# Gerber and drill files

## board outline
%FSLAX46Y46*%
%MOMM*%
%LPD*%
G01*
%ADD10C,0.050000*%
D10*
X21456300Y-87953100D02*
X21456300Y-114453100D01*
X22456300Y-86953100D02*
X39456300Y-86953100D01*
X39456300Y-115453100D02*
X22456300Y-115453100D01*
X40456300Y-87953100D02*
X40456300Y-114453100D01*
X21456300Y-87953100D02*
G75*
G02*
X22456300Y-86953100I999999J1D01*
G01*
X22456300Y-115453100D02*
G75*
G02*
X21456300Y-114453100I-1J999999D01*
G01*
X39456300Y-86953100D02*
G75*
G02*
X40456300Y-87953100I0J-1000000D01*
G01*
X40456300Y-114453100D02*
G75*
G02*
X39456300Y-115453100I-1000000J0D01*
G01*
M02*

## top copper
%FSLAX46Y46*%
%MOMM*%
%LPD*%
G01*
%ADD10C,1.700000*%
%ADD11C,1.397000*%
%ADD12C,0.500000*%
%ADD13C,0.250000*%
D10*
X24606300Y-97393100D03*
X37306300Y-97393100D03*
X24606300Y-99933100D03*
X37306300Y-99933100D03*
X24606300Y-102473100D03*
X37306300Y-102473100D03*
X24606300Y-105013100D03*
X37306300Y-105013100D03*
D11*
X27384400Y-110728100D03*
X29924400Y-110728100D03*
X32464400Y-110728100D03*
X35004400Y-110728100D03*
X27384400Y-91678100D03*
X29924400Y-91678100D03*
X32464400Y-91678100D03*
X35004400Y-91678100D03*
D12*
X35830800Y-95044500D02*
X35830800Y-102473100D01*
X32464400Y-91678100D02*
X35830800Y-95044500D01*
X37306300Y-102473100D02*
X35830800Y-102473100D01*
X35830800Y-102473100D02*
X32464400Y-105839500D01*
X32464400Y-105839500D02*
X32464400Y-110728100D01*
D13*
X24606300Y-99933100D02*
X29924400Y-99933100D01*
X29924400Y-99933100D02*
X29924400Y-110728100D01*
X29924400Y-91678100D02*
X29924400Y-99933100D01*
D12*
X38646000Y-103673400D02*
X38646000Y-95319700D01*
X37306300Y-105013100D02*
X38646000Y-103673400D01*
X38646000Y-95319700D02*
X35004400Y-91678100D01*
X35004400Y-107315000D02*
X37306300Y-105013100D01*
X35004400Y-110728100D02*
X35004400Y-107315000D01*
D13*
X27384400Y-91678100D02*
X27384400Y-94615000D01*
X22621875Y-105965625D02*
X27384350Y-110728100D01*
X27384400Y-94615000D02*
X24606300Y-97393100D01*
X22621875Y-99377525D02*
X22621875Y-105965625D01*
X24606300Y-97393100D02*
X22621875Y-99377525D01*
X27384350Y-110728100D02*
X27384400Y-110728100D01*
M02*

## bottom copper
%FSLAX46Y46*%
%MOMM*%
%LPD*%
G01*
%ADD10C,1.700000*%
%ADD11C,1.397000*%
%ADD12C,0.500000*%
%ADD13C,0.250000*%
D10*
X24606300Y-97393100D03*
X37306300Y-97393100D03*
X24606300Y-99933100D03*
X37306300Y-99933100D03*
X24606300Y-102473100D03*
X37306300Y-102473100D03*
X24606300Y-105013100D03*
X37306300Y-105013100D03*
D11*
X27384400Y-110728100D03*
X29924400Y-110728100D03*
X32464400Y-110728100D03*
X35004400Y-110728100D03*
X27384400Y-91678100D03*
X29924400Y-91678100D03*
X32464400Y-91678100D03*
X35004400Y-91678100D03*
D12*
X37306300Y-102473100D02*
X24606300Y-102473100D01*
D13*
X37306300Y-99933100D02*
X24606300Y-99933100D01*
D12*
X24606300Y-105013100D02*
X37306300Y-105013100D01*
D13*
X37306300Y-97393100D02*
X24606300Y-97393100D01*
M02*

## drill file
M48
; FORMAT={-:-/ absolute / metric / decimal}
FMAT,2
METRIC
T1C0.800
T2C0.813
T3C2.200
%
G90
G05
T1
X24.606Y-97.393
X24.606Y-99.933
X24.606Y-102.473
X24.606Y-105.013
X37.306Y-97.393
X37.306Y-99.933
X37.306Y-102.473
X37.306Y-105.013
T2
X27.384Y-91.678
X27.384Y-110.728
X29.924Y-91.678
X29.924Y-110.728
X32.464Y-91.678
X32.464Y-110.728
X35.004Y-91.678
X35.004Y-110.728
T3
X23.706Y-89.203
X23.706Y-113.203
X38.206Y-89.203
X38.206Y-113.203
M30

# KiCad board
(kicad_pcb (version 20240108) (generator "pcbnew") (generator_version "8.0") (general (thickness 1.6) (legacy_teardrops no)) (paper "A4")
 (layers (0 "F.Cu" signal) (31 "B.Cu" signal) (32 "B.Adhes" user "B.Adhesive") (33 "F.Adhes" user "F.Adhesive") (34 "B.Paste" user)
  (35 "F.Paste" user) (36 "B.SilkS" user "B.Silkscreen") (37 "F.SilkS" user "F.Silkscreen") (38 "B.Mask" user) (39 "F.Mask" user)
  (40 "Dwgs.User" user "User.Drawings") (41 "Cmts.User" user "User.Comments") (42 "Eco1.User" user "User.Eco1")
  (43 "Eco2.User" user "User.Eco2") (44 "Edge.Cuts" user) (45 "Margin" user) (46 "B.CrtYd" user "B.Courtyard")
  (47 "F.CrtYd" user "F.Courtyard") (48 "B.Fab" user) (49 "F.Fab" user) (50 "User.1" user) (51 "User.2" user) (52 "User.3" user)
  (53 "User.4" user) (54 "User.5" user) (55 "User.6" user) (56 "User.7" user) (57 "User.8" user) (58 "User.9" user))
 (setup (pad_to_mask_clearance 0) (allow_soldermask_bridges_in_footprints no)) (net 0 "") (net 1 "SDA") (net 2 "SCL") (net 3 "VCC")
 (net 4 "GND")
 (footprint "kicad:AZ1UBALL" (layer "F.Cu") (at 30.9563 101.2031)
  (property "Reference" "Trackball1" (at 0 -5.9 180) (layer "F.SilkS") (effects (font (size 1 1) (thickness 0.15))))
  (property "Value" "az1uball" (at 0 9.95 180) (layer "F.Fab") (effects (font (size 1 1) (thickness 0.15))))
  (pad "1" thru_hole circle (at -6.35 -3.81) (size 1.7 1.7) (drill 0.8) (layers "*.Cu" "*.Mask") (remove_unused_layers no) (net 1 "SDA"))
  (pad "1" thru_hole circle (at 6.35 -3.81) (size 1.7 1.7) (drill 0.8) (layers "*.Cu" "*.Mask") (remove_unused_layers no) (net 1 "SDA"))
  (pad "2" thru_hole circle (at -6.35 -1.27) (size 1.7 1.7) (drill 0.8) (layers "*.Cu" "*.Mask") (remove_unused_layers no) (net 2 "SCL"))
  (pad "2" thru_hole circle (at 6.35 -1.27) (size 1.7 1.7) (drill 0.8) (layers "*.Cu" "*.Mask") (remove_unused_layers no) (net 2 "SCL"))
  (pad "3" thru_hole circle (at -6.35 1.27) (size 1.7 1.7) (drill 0.8) (layers "*.Cu" "*.Mask") (remove_unused_layers no) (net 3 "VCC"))
  (pad "3" thru_hole circle (at 6.35 1.27) (size 1.7 1.7) (drill 0.8) (layers "*.Cu" "*.Mask") (remove_unused_layers no) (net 3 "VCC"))
  (pad "4" thru_hole circle (at -6.35 3.81) (size 1.7 1.7) (drill 0.8) (layers "*.Cu" "*.Mask") (remove_unused_layers no) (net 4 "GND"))
  (pad "4" thru_hole circle (at 6.35 3.81) (size 1.7 1.7) (drill 0.8) (layers "*.Cu" "*.Mask") (remove_unused_layers no) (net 4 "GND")))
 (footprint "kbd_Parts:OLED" (layer "F.Cu") (at 27.3844 110.7281)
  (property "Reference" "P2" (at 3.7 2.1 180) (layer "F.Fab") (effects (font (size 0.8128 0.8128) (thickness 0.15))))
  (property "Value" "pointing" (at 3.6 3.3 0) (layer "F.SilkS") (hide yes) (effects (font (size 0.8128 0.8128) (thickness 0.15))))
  (pad "1" thru_hole circle (at 0 0) (size 1.397 1.397) (drill 0.8128) (layers "*.Cu" "*.Mask" "F.SilkS") (remove_unused_layers no)
   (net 1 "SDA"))
  (pad "2" thru_hole circle (at 2.54 0) (size 1.397 1.397) (drill 0.8128) (layers "*.Cu" "*.Mask" "F.SilkS") (remove_unused_layers no)
   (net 2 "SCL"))
  (pad "3" thru_hole circle (at 5.08 0) (size 1.397 1.397) (drill 0.8128) (layers "*.Cu" "*.Mask" "F.SilkS") (remove_unused_layers no)
   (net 3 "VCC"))
  (pad "4" thru_hole circle (at 7.62 0) (size 1.397 1.397) (drill 0.8128) (layers "*.Cu" "*.Mask" "F.SilkS") (remove_unused_layers no)
   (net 4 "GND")))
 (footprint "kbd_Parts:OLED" (layer "F.Cu") (at 27.3844 91.6781)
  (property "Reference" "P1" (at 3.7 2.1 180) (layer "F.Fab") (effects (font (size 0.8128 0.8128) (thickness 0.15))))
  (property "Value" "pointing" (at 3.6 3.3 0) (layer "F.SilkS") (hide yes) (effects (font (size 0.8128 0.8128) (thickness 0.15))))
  (pad "1" thru_hole circle (at 0 0) (size 1.397 1.397) (drill 0.8128) (layers "*.Cu" "*.Mask" "F.SilkS") (remove_unused_layers no)
   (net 1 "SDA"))
  (pad "2" thru_hole circle (at 2.54 0) (size 1.397 1.397) (drill 0.8128) (layers "*.Cu" "*.Mask" "F.SilkS") (remove_unused_layers no)
   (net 2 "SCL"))
  (pad "3" thru_hole circle (at 5.08 0) (size 1.397 1.397) (drill 0.8128) (layers "*.Cu" "*.Mask" "F.SilkS") (remove_unused_layers no)
   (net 3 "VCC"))
  (pad "4" thru_hole circle (at 7.62 0) (size 1.397 1.397) (drill 0.8128) (layers "*.Cu" "*.Mask" "F.SilkS") (remove_unused_layers no)
   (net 4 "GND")))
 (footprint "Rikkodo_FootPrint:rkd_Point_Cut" (layer "F.Cu") (at 30.9563 101.2031)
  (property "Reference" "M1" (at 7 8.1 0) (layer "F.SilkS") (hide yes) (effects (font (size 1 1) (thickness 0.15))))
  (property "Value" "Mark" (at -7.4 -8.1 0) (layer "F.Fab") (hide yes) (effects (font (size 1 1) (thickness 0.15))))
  (fp_line (start -9.5 -13.25) (end -9.5 13.25) (stroke (width 0.05) (type default)) (layer "Edge.Cuts"))
  (fp_line (start -8.5 -14.25) (end 8.5 -14.25) (stroke (width 0.05) (type default)) (layer "Edge.Cuts"))
  (fp_line (start 8.5 14.25) (end -8.5 14.25) (stroke (width 0.05) (type default)) (layer "Edge.Cuts"))
  (fp_line (start 9.5 -13.25) (end 9.5 13.25) (stroke (width 0.05) (type default)) (layer "Edge.Cuts"))
  (fp_arc (start -9.5 -13.25) (mid -9.207107 -13.957107) (end -8.5 -14.25) (stroke (width 0.05) (type default)) (layer "Edge.Cuts"))
  (fp_arc (start -8.5 14.25) (mid -9.207107 13.957107) (end -9.5 13.25) (stroke (width 0.05) (type default)) (layer "Edge.Cuts"))
  (fp_arc (start 8.5 -14.25) (mid 9.207107 -13.957107) (end 9.5 -13.25) (stroke (width 0.05) (type default)) (layer "Edge.Cuts"))
  (fp_arc (start 9.5 13.25) (mid 9.207107 13.957107) (end 8.5 14.25) (stroke (width 0.05) (type default)) (layer "Edge.Cuts"))
  (pad "" np_thru_hole circle (at -7.25 -12) (size 2.2 2.2) (drill 2.2) (layers "*.Cu" "*.Mask"))
  (pad "" np_thru_hole circle (at -7.25 12) (size 2.2 2.2) (drill 2.2) (layers "*.Cu" "*.Mask"))
  (pad "" np_thru_hole circle (at 7.25 -12) (size 2.2 2.2) (drill 2.2) (layers "*.Cu" "*.Mask"))
  (pad "" np_thru_hole circle (at 7.25 12) (size 2.2 2.2) (drill 2.2) (layers "*.Cu" "*.Mask")))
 (segment (start 35.8308 95.0445) (end 35.8308 102.4731) (width 0.5) (layer "F.Cu") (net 3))
 (segment (start 32.4644 91.6781) (end 35.8308 95.0445) (width 0.5) (layer "F.Cu") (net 3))
 (segment (start 37.3063 102.4731) (end 35.8308 102.4731) (width 0.5) (layer "F.Cu") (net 3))
 (segment (start 35.8308 102.4731) (end 32.4644 105.8395) (width 0.5) (layer "F.Cu") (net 3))
 (segment (start 32.4644 105.8395) (end 32.4644 110.7281) (width 0.5) (layer "F.Cu") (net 3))
 (segment (start 37.3063 102.4731) (end 24.6063 102.4731) (width 0.5) (layer "B.Cu") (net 3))
 (segment (start 24.6063 99.9331) (end 29.9244 99.9331) (width 0.25) (layer "F.Cu") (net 2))
 (segment (start 29.9244 99.9331) (end 29.9244 110.7281) (width 0.25) (layer "F.Cu") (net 2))
 (segment (start 29.9244 91.6781) (end 29.9244 99.9331) (width 0.25) (layer "F.Cu") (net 2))
 (segment (start 37.3063 99.9331) (end 24.6063 99.9331) (width 0.25) (layer "B.Cu") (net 2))
 (segment (start 38.646 103.6734) (end 38.646 95.3197) (width 0.5) (layer "F.Cu") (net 4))
 (segment (start 37.3063 105.0131) (end 38.646 103.6734) (width 0.5) (layer "F.Cu") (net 4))
 (segment (start 38.646 95.3197) (end 35.0044 91.6781) (width 0.5) (layer "F.Cu") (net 4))
 (segment (start 35.0044 107.315) (end 37.3063 105.0131) (width 0.5) (layer "F.Cu") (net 4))
 (segment (start 35.0044 110.7281) (end 35.0044 107.315) (width 0.5) (layer "F.Cu") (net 4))
 (segment (start 24.6063 105.0131) (end 37.3063 105.0131) (width 0.5) (layer "B.Cu") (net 4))
 (segment (start 27.3844 91.6781) (end 27.3844 94.615) (width 0.25) (layer "F.Cu") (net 1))
 (segment (start 22.621875 105.965625) (end 27.38435 110.7281) (width 0.25) (layer "F.Cu") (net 1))
 (segment (start 27.3844 94.615) (end 24.6063 97.3931) (width 0.25) (layer "F.Cu") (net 1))
 (segment (start 22.621875 99.377525) (end 22.621875 105.965625) (width 0.25) (layer "F.Cu") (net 1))
 (segment (start 24.6063 97.3931) (end 22.621875 99.377525) (width 0.25) (layer "F.Cu") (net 1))
 (segment (start 27.38435 110.7281) (end 27.3844 110.7281) (width 0.25) (layer "F.Cu") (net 1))
 (segment (start 37.3063 97.3931) (end 24.6063 97.3931) (width 0.25) (layer "B.Cu") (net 1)))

